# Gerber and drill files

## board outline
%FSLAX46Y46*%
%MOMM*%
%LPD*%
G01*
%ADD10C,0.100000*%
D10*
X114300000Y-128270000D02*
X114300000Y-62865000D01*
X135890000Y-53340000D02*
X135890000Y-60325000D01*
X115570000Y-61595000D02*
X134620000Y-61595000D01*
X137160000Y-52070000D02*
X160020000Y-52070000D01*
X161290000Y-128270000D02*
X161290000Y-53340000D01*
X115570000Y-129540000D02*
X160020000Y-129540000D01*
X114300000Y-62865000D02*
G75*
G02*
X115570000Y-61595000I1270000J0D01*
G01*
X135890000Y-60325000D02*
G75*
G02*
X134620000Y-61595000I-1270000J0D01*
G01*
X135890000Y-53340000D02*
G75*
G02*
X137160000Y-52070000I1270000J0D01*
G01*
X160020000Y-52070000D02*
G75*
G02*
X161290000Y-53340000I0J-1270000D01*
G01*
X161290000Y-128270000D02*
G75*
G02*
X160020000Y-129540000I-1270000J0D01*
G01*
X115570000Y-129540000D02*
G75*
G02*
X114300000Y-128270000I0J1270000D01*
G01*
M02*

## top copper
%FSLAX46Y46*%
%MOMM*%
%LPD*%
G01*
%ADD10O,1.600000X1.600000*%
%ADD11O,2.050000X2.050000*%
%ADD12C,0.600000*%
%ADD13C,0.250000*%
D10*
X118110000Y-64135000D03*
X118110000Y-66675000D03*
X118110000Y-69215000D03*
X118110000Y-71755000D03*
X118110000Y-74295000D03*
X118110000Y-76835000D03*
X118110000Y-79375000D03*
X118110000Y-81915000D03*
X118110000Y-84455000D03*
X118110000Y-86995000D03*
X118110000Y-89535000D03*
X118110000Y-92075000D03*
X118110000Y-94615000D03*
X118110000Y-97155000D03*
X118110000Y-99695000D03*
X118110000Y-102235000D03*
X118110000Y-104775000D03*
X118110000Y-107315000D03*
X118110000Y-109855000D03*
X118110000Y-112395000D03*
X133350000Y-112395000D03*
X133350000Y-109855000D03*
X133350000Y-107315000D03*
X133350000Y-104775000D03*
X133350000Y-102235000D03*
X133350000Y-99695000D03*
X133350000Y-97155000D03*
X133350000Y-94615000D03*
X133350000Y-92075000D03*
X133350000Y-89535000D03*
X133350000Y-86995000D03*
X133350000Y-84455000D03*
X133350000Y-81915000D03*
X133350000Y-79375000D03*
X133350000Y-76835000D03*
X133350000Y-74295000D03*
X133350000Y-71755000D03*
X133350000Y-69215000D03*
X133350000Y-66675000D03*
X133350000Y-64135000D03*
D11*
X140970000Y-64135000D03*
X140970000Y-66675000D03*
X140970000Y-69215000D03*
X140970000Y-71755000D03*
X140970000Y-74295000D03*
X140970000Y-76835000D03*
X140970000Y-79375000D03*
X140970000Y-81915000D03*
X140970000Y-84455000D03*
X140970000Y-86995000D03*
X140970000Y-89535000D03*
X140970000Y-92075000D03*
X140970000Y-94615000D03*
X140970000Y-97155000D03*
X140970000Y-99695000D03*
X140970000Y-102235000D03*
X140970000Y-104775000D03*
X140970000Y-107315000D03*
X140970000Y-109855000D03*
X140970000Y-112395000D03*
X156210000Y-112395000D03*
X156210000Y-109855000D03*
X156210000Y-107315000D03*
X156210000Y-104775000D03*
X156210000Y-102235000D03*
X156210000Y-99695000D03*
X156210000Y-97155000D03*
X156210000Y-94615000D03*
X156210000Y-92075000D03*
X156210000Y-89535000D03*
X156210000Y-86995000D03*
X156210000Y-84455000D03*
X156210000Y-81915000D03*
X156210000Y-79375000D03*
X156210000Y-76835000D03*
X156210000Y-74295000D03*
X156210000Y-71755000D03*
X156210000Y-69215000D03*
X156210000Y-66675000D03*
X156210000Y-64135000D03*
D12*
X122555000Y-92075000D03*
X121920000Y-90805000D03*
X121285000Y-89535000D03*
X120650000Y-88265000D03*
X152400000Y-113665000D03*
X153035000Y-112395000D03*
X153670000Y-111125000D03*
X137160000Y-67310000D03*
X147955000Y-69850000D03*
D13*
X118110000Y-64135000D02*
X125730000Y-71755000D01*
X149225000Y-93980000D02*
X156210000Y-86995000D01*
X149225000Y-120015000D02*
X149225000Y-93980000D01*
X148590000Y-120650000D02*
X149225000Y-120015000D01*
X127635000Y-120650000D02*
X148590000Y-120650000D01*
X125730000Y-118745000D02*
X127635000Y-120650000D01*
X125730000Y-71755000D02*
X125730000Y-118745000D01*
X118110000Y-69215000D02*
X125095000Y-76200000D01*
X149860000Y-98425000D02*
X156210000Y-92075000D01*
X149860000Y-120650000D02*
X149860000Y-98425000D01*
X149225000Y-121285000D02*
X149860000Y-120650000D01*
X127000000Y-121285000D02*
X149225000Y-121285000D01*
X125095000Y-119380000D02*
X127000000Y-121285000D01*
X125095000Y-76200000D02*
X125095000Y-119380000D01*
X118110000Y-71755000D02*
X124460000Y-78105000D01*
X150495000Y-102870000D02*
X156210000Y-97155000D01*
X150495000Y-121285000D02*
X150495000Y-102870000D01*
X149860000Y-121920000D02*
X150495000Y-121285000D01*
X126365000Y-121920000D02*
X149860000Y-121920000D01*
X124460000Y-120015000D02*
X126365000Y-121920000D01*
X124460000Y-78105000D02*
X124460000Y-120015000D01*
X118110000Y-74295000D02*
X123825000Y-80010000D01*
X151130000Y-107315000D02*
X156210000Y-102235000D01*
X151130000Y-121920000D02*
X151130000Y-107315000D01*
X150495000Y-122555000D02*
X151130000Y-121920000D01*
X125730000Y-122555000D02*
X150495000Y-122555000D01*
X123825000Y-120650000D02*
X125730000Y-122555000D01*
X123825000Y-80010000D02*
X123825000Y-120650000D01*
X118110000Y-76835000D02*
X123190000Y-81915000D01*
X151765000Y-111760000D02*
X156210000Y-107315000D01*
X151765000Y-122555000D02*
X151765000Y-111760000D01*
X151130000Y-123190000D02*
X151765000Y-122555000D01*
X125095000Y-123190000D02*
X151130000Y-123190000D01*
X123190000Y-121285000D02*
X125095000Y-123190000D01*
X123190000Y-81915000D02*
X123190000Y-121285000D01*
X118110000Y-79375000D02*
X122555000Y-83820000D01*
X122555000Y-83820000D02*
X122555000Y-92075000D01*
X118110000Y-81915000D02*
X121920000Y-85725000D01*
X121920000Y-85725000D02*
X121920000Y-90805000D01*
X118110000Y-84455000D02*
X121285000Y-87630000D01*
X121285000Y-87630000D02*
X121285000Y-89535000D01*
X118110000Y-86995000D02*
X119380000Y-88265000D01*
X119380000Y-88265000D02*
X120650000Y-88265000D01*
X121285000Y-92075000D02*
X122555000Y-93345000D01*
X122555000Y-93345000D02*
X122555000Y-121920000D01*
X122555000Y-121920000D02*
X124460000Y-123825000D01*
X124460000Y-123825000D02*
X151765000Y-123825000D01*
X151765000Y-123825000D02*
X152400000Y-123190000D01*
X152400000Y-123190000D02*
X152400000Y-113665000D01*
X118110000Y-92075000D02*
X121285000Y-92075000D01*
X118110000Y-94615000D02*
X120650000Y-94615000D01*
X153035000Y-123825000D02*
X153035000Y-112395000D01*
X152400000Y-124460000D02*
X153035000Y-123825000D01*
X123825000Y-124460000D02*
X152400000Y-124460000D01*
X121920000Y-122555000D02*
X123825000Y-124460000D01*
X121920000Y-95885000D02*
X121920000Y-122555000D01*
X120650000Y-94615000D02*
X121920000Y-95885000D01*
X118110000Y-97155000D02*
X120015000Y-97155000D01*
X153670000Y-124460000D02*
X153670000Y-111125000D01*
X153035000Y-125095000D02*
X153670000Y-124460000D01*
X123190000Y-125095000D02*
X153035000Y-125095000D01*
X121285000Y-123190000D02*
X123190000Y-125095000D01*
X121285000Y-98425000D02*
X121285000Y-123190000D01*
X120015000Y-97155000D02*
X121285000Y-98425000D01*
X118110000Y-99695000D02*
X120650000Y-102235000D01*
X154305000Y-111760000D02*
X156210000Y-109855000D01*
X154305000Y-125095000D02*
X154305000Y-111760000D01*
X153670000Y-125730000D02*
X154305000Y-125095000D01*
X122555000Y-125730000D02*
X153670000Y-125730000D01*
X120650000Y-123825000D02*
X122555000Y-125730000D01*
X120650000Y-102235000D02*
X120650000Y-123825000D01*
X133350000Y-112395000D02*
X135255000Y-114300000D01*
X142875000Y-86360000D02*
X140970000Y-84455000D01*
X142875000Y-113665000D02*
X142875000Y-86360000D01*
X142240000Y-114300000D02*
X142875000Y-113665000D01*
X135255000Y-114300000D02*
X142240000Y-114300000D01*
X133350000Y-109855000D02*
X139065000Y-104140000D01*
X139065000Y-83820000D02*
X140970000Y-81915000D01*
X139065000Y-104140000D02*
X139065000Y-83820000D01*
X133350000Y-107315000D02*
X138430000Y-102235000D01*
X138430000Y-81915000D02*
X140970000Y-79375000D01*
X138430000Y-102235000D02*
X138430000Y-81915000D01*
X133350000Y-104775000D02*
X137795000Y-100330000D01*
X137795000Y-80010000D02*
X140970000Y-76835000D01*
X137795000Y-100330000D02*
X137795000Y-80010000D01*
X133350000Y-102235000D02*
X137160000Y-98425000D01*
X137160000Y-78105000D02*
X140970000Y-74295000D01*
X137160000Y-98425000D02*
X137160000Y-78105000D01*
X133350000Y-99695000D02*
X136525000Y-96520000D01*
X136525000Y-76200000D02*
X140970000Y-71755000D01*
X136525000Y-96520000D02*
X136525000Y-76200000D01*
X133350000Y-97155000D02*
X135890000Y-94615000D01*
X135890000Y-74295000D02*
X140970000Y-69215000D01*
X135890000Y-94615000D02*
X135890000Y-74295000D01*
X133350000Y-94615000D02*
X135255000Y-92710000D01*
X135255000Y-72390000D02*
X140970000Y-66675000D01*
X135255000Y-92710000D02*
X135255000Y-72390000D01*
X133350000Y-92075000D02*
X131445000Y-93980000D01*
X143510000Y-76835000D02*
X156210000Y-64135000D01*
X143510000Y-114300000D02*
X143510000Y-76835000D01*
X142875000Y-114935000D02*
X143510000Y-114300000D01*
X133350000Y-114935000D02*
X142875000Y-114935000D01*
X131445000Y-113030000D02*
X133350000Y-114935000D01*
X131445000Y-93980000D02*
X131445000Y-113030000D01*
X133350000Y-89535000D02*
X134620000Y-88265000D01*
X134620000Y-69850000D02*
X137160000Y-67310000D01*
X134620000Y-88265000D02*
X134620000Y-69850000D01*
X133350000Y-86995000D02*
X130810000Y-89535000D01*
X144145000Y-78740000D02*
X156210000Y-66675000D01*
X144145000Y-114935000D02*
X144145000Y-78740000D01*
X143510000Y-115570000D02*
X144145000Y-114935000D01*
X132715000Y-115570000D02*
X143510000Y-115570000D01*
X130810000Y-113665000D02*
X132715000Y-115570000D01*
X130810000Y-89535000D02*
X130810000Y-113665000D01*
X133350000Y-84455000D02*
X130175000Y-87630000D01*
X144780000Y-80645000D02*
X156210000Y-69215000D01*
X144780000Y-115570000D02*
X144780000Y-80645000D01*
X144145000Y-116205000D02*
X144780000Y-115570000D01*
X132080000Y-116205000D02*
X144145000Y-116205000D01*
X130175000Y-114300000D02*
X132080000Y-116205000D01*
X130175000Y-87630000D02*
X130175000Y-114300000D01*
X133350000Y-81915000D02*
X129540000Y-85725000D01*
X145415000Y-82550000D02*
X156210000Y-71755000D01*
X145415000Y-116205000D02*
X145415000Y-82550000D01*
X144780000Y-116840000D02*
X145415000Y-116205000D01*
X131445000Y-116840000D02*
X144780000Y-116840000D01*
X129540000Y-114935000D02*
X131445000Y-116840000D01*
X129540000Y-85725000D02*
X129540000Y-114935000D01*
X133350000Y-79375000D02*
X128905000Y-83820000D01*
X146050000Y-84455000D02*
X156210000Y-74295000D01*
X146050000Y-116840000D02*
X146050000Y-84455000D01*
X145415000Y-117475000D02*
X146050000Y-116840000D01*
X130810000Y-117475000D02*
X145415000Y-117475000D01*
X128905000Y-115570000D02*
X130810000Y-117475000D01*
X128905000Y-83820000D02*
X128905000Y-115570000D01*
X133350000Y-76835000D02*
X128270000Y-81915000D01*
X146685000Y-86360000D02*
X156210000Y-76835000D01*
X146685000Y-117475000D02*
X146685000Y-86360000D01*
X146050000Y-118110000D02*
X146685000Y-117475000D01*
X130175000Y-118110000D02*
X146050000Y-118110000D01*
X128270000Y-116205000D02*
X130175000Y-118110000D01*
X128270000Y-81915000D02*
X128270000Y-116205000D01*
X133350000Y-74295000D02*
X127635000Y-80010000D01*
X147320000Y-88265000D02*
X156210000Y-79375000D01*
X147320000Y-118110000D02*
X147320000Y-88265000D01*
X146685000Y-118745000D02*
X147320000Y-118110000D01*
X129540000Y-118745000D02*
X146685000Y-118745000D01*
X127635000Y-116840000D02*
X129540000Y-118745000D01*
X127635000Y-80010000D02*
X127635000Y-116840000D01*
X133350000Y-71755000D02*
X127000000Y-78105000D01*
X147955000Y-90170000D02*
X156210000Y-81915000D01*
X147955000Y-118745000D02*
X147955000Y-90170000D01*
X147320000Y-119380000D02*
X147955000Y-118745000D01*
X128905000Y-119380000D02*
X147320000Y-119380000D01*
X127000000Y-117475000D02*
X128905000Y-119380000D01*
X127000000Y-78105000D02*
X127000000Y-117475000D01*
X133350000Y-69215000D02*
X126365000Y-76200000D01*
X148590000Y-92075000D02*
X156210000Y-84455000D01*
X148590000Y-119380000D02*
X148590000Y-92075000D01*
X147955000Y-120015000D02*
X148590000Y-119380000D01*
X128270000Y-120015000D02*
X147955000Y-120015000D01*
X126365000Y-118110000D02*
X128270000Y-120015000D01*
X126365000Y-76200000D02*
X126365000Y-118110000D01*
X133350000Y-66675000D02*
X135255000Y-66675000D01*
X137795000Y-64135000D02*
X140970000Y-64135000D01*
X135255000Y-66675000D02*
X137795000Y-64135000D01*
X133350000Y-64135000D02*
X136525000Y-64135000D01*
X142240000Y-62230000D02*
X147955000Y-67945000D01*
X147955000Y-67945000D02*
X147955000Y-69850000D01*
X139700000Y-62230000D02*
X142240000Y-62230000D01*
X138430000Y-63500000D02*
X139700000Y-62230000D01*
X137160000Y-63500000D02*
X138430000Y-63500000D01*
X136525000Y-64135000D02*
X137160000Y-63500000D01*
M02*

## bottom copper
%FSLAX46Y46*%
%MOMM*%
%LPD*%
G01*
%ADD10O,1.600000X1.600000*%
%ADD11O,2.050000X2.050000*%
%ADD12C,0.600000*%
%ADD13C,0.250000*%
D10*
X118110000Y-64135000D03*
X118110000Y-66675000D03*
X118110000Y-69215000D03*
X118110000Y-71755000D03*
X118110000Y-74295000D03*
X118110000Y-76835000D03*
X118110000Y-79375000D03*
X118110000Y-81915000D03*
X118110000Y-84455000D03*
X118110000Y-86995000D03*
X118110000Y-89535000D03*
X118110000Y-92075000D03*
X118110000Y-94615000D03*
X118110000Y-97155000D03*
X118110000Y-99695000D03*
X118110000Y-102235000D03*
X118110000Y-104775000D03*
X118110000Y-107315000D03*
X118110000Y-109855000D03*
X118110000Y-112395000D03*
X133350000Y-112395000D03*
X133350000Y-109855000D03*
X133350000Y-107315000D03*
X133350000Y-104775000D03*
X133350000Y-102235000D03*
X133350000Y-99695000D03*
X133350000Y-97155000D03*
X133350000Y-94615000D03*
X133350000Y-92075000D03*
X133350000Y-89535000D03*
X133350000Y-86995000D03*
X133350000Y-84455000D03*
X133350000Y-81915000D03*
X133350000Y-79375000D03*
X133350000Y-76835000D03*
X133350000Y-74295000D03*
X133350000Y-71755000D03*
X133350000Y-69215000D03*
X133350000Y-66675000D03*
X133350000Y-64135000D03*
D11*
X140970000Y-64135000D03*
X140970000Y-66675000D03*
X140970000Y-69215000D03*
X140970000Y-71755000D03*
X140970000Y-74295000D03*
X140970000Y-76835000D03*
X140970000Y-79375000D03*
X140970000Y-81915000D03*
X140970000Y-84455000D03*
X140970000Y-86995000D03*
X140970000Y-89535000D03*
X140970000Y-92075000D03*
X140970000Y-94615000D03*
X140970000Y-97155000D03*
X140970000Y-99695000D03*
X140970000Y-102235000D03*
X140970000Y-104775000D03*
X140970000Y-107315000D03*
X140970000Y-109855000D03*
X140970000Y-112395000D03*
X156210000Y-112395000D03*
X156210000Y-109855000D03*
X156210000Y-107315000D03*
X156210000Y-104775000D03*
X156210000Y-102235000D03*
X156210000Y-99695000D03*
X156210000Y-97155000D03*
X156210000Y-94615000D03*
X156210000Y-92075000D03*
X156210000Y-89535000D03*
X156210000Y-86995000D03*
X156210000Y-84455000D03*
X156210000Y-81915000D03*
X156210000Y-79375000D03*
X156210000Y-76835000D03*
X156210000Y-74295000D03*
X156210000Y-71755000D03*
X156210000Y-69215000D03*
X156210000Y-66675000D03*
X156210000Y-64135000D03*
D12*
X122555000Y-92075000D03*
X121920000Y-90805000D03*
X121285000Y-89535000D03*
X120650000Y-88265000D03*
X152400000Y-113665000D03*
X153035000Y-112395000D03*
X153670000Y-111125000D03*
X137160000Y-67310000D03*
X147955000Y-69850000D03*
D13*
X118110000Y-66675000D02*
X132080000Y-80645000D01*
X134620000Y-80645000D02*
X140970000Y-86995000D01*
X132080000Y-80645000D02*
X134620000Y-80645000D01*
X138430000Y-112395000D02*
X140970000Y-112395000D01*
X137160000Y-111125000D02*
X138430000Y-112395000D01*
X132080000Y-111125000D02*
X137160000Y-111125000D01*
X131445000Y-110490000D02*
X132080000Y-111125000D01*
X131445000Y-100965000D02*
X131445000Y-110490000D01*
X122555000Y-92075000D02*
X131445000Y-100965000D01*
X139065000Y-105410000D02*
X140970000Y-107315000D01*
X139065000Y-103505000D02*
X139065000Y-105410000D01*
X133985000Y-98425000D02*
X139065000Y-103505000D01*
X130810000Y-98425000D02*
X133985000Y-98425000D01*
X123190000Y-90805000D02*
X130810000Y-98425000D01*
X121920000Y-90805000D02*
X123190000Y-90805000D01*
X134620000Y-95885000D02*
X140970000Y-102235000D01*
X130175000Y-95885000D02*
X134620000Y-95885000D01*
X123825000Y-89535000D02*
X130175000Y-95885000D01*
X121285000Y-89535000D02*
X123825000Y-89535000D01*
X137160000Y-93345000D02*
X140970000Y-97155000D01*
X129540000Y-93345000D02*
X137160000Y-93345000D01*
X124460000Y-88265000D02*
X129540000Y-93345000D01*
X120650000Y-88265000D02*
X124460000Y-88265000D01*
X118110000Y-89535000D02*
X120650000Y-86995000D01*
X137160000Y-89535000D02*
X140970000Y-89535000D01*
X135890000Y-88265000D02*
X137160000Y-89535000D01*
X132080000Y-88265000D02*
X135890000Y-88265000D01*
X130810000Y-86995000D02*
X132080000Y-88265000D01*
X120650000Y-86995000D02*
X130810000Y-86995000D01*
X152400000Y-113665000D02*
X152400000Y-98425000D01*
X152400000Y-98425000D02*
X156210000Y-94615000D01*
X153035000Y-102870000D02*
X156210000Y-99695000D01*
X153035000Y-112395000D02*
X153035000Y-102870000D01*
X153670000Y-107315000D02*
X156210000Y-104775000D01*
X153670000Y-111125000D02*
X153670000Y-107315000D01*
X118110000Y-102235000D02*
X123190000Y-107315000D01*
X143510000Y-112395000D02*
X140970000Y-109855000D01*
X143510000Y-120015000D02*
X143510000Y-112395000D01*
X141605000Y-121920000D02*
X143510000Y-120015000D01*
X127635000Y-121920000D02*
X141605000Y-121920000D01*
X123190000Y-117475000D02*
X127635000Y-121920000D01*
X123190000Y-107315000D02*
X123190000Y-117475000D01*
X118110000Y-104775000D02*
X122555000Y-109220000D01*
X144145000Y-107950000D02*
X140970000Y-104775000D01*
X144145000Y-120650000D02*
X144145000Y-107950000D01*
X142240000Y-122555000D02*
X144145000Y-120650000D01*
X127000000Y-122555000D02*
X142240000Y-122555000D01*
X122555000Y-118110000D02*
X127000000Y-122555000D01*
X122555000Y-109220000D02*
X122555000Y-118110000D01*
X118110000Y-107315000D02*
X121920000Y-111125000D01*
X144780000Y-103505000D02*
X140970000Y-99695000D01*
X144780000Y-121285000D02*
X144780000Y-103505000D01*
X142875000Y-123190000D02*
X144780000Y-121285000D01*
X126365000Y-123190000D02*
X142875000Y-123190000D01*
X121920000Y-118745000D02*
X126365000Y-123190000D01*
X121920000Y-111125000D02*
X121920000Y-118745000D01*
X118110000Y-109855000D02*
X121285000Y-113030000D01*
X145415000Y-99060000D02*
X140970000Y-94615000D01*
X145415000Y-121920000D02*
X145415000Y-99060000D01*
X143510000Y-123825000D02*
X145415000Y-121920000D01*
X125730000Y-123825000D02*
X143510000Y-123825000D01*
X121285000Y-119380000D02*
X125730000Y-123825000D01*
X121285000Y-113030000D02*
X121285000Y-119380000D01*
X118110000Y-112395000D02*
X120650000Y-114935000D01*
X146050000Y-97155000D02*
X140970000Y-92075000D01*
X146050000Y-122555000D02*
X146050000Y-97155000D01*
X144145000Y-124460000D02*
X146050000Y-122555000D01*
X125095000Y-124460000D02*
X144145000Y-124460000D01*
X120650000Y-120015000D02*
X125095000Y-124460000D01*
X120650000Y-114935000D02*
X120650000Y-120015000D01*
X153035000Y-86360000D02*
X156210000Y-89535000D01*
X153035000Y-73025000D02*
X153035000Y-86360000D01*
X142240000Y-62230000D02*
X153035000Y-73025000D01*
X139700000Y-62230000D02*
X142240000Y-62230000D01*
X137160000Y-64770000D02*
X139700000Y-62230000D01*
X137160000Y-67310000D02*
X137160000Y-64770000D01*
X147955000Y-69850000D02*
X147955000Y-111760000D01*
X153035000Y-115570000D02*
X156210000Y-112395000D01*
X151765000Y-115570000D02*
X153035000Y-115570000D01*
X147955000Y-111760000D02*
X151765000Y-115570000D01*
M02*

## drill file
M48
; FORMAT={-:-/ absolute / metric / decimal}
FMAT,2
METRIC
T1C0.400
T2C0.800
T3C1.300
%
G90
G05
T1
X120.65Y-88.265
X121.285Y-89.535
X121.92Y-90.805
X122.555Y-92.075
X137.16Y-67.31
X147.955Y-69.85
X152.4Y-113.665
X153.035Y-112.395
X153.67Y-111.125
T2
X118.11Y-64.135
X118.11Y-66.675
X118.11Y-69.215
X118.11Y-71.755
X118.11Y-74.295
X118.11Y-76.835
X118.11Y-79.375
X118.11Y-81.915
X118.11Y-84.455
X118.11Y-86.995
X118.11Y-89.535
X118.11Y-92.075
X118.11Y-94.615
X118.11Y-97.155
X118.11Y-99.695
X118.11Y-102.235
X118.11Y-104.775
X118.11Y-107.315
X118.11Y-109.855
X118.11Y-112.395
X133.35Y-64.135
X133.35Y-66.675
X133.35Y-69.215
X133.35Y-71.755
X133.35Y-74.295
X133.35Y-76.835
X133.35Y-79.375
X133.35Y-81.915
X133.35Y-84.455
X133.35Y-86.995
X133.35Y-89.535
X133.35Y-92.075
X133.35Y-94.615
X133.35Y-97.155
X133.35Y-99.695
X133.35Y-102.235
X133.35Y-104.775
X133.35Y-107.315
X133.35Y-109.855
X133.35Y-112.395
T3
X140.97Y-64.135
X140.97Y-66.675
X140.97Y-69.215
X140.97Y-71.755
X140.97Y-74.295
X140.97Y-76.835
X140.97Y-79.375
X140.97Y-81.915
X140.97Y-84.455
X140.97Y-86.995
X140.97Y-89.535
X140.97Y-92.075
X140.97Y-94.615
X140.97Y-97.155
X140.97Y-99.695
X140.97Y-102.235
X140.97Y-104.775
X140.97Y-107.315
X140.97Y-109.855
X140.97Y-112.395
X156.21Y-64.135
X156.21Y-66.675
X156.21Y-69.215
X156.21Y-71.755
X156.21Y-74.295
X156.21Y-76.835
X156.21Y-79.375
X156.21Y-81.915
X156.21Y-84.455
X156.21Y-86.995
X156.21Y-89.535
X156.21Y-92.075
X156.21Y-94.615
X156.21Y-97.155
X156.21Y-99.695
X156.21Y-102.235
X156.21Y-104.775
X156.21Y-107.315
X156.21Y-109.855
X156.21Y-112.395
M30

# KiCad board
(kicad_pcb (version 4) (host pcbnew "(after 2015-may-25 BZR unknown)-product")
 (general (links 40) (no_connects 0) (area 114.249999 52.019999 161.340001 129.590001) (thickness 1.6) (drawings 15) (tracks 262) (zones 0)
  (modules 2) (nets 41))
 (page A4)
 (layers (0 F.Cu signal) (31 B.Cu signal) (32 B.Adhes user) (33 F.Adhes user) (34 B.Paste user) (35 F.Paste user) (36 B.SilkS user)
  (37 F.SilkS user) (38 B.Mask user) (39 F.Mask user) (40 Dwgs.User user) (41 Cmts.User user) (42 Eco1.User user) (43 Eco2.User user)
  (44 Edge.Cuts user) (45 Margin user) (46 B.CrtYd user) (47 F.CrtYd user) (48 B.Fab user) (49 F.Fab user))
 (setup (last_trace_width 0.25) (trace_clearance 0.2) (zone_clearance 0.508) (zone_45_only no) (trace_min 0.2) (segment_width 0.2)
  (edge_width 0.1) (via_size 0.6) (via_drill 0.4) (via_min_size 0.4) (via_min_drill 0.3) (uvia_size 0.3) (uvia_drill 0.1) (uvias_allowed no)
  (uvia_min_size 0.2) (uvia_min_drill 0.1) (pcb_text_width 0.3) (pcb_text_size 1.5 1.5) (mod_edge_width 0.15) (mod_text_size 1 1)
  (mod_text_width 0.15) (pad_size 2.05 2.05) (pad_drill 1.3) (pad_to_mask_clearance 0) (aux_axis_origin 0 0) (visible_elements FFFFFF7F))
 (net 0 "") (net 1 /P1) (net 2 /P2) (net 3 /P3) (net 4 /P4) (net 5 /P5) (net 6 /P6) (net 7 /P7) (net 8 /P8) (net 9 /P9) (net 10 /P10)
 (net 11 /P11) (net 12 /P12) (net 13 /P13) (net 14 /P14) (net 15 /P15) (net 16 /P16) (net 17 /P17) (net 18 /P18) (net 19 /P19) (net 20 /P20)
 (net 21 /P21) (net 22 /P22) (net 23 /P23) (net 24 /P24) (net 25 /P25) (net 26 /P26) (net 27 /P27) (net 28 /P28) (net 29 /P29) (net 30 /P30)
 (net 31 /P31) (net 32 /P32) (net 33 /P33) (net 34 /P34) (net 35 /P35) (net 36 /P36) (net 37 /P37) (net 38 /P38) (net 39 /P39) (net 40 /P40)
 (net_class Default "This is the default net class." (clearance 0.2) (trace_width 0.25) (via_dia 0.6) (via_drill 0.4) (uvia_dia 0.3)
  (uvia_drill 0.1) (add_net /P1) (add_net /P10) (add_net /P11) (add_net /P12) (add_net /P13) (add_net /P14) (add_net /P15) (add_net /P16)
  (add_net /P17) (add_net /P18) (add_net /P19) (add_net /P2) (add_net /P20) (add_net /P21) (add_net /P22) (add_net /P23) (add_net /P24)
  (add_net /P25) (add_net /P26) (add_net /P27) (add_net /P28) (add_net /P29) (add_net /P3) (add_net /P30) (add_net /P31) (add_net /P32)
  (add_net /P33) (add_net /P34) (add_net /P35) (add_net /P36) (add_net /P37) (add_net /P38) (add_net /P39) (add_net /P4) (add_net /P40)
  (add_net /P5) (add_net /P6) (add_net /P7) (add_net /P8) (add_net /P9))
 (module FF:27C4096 (layer F.Cu) (at 118.11 64.135)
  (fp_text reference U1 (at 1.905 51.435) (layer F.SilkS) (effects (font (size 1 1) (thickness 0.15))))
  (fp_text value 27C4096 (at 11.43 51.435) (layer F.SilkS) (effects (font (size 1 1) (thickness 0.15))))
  (pad 1 thru_hole oval (at 0 0) (size 1.6 1.6) (drill 0.8) (layers *.Cu *.Mask F.SilkS) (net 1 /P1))
  (pad 2 thru_hole oval (at 0 2.54) (size 1.6 1.6) (drill 0.8) (layers *.Cu *.Mask F.SilkS) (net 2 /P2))
  (pad 3 thru_hole oval (at 0 5.08) (size 1.6 1.6) (drill 0.8) (layers *.Cu *.Mask F.SilkS) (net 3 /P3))
  (pad 4 thru_hole oval (at 0 7.62) (size 1.6 1.6) (drill 0.8) (layers *.Cu *.Mask F.SilkS) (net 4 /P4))
  (pad 5 thru_hole oval (at 0 10.16) (size 1.6 1.6) (drill 0.8) (layers *.Cu *.Mask F.SilkS) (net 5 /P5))
  (pad 6 thru_hole oval (at 0 12.7) (size 1.6 1.6) (drill 0.8) (layers *.Cu *.Mask F.SilkS) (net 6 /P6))
  (pad 7 thru_hole oval (at 0 15.24) (size 1.6 1.6) (drill 0.8) (layers *.Cu *.Mask F.SilkS) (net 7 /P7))
  (pad 8 thru_hole oval (at 0 17.78) (size 1.6 1.6) (drill 0.8) (layers *.Cu *.Mask F.SilkS) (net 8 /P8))
  (pad 9 thru_hole oval (at 0 20.32) (size 1.6 1.6) (drill 0.8) (layers *.Cu *.Mask F.SilkS) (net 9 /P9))
  (pad 10 thru_hole oval (at 0 22.86) (size 1.6 1.6) (drill 0.8) (layers *.Cu *.Mask F.SilkS) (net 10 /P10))
  (pad 11 thru_hole oval (at 0 25.4) (size 1.6 1.6) (drill 0.8) (layers *.Cu *.Mask F.SilkS) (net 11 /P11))
  (pad 12 thru_hole oval (at 0 27.94) (size 1.6 1.6) (drill 0.8) (layers *.Cu *.Mask F.SilkS) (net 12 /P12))
  (pad 13 thru_hole oval (at 0 30.48) (size 1.6 1.6) (drill 0.8) (layers *.Cu *.Mask F.SilkS) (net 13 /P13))
  (pad 14 thru_hole oval (at 0 33.02) (size 1.6 1.6) (drill 0.8) (layers *.Cu *.Mask F.SilkS) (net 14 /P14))
  (pad 15 thru_hole oval (at 0 35.56) (size 1.6 1.6) (drill 0.8) (layers *.Cu *.Mask F.SilkS) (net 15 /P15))
  (pad 16 thru_hole oval (at 0 38.1) (size 1.6 1.6) (drill 0.8) (layers *.Cu *.Mask F.SilkS) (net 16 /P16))
  (pad 17 thru_hole oval (at 0 40.64) (size 1.6 1.6) (drill 0.8) (layers *.Cu *.Mask F.SilkS) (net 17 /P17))
  (pad 18 thru_hole oval (at 0 43.18) (size 1.6 1.6) (drill 0.8) (layers *.Cu *.Mask F.SilkS) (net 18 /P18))
  (pad 19 thru_hole oval (at 0 45.72) (size 1.6 1.6) (drill 0.8) (layers *.Cu *.Mask F.SilkS) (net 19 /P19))
  (pad 20 thru_hole oval (at 0 48.26) (size 1.6 1.6) (drill 0.8) (layers *.Cu *.Mask F.SilkS) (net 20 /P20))
  (pad 21 thru_hole oval (at 15.24 48.26) (size 1.6 1.6) (drill 0.8) (layers *.Cu *.Mask F.SilkS) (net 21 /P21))
  (pad 22 thru_hole oval (at 15.24 45.72) (size 1.6 1.6) (drill 0.8) (layers *.Cu *.Mask F.SilkS) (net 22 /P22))
  (pad 23 thru_hole oval (at 15.24 43.18) (size 1.6 1.6) (drill 0.8) (layers *.Cu *.Mask F.SilkS) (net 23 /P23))
  (pad 24 thru_hole oval (at 15.24 40.64) (size 1.6 1.6) (drill 0.8) (layers *.Cu *.Mask F.SilkS) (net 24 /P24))
  (pad 25 thru_hole oval (at 15.24 38.1) (size 1.6 1.6) (drill 0.8) (layers *.Cu *.Mask F.SilkS) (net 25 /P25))
  (pad 26 thru_hole oval (at 15.24 35.56) (size 1.6 1.6) (drill 0.8) (layers *.Cu *.Mask F.SilkS) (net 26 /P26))
  (pad 27 thru_hole oval (at 15.24 33.02) (size 1.6 1.6) (drill 0.8) (layers *.Cu *.Mask F.SilkS) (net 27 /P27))
  (pad 28 thru_hole oval (at 15.24 30.48) (size 1.6 1.6) (drill 0.8) (layers *.Cu *.Mask F.SilkS) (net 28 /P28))
  (pad 29 thru_hole oval (at 15.24 27.94) (size 1.6 1.6) (drill 0.8) (layers *.Cu *.Mask F.SilkS) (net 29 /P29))
  (pad 30 thru_hole oval (at 15.24 25.4) (size 1.6 1.6) (drill 0.8) (layers *.Cu *.Mask F.SilkS) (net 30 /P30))
  (pad 31 thru_hole oval (at 15.24 22.86) (size 1.6 1.6) (drill 0.8) (layers *.Cu *.Mask F.SilkS) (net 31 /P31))
  (pad 32 thru_hole oval (at 15.24 20.32) (size 1.6 1.6) (drill 0.8) (layers *.Cu *.Mask F.SilkS) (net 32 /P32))
  (pad 33 thru_hole oval (at 15.24 17.78) (size 1.6 1.6) (drill 0.8) (layers *.Cu *.Mask F.SilkS) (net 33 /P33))
  (pad 34 thru_hole oval (at 15.24 15.24) (size 1.6 1.6) (drill 0.8) (layers *.Cu *.Mask F.SilkS) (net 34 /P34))
  (pad 35 thru_hole oval (at 15.24 12.7) (size 1.6 1.6) (drill 0.8) (layers *.Cu *.Mask F.SilkS) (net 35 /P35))
  (pad 36 thru_hole oval (at 15.24 10.16) (size 1.6 1.6) (drill 0.8) (layers *.Cu *.Mask F.SilkS) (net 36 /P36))
  (pad 37 thru_hole oval (at 15.24 7.62) (size 1.6 1.6) (drill 0.8) (layers *.Cu *.Mask F.SilkS) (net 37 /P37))
  (pad 38 thru_hole oval (at 15.24 5.08) (size 1.6 1.6) (drill 0.8) (layers *.Cu *.Mask F.SilkS) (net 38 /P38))
  (pad 39 thru_hole oval (at 15.24 2.54) (size 1.6 1.6) (drill 0.8) (layers *.Cu *.Mask F.SilkS) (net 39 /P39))
  (pad 40 thru_hole oval (at 15.24 0) (size 1.6 1.6) (drill 0.8) (layers *.Cu *.Mask F.SilkS) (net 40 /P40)))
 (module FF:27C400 (layer F.Cu) (at 140.97 64.135)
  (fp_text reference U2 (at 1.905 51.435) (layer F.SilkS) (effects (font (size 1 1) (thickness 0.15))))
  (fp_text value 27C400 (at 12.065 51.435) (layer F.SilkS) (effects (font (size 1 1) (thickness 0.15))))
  (pad 1 thru_hole oval (at 0 0) (size 2.05 2.05) (drill 1.3) (layers *.Cu *.Mask F.SilkS) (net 39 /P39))
  (pad 2 thru_hole oval (at 0 2.54) (size 2.05 2.05) (drill 1.3) (layers *.Cu *.Mask F.SilkS) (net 28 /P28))
  (pad 3 thru_hole oval (at 0 5.08) (size 2.05 2.05) (drill 1.3) (layers *.Cu *.Mask F.SilkS) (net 27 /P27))
  (pad 4 thru_hole oval (at 0 7.62) (size 2.05 2.05) (drill 1.3) (layers *.Cu *.Mask F.SilkS) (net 26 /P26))
  (pad 5 thru_hole oval (at 0 10.16) (size 2.05 2.05) (drill 1.3) (layers *.Cu *.Mask F.SilkS) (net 25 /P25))
  (pad 6 thru_hole oval (at 0 12.7) (size 2.05 2.05) (drill 1.3) (layers *.Cu *.Mask F.SilkS) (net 24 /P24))
  (pad 7 thru_hole oval (at 0 15.24) (size 2.05 2.05) (drill 1.3) (layers *.Cu *.Mask F.SilkS) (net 23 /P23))
  (pad 8 thru_hole oval (at 0 17.78) (size 2.05 2.05) (drill 1.3) (layers *.Cu *.Mask F.SilkS) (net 22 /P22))
  (pad 9 thru_hole oval (at 0 20.32) (size 2.05 2.05) (drill 1.3) (layers *.Cu *.Mask F.SilkS) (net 21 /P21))
  (pad 10 thru_hole oval (at 0 22.86) (size 2.05 2.05) (drill 1.3) (layers *.Cu *.Mask F.SilkS) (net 2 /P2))
  (pad 11 thru_hole oval (at 0 25.4) (size 2.05 2.05) (drill 1.3) (layers *.Cu *.Mask F.SilkS) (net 11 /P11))
  (pad 12 thru_hole oval (at 0 27.94) (size 2.05 2.05) (drill 1.3) (layers *.Cu *.Mask F.SilkS) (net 20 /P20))
  (pad 13 thru_hole oval (at 0 30.48) (size 2.05 2.05) (drill 1.3) (layers *.Cu *.Mask F.SilkS) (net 19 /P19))
  (pad 14 thru_hole oval (at 0 33.02) (size 2.05 2.05) (drill 1.3) (layers *.Cu *.Mask F.SilkS) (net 10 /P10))
  (pad 15 thru_hole oval (at 0 35.56) (size 2.05 2.05) (drill 1.3) (layers *.Cu *.Mask F.SilkS) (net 18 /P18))
  (pad 16 thru_hole oval (at 0 38.1) (size 2.05 2.05) (drill 1.3) (layers *.Cu *.Mask F.SilkS) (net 9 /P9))
  (pad 17 thru_hole oval (at 0 40.64) (size 2.05 2.05) (drill 1.3) (layers *.Cu *.Mask F.SilkS) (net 17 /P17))
  (pad 18 thru_hole oval (at 0 43.18) (size 2.05 2.05) (drill 1.3) (layers *.Cu *.Mask F.SilkS) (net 8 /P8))
  (pad 19 thru_hole oval (at 0 45.72) (size 2.05 2.05) (drill 1.3) (layers *.Cu *.Mask F.SilkS) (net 16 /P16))
  (pad 20 thru_hole oval (at 0 48.26) (size 2.05 2.05) (drill 1.3) (layers *.Cu *.Mask F.SilkS) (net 7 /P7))
  (pad 21 thru_hole oval (at 15.24 48.26) (size 2.05 2.05) (drill 1.3) (layers *.Cu *.Mask F.SilkS) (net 40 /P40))
  (pad 22 thru_hole oval (at 15.24 45.72) (size 2.05 2.05) (drill 1.3) (layers *.Cu *.Mask F.SilkS) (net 15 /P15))
  (pad 23 thru_hole oval (at 15.24 43.18) (size 2.05 2.05) (drill 1.3) (layers *.Cu *.Mask F.SilkS) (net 6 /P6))
  (pad 24 thru_hole oval (at 15.24 40.64) (size 2.05 2.05) (drill 1.3) (layers *.Cu *.Mask F.SilkS) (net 14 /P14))
  (pad 25 thru_hole oval (at 15.24 38.1) (size 2.05 2.05) (drill 1.3) (layers *.Cu *.Mask F.SilkS) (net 5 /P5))
  (pad 26 thru_hole oval (at 15.24 35.56) (size 2.05 2.05) (drill 1.3) (layers *.Cu *.Mask F.SilkS) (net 13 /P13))
  (pad 27 thru_hole oval (at 15.24 33.02) (size 2.05 2.05) (drill 1.3) (layers *.Cu *.Mask F.SilkS) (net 4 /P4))
  (pad 28 thru_hole oval (at 15.24 30.48) (size 2.05 2.05) (drill 1.3) (layers *.Cu *.Mask F.SilkS) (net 12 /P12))
  (pad 29 thru_hole oval (at 15.24 27.94) (size 2.05 2.05) (drill 1.3) (layers *.Cu *.Mask F.SilkS) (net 3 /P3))
  (pad 30 thru_hole oval (at 15.24 25.4) (size 2.05 2.05) (drill 1.3) (layers *.Cu *.Mask F.SilkS) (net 30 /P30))
  (pad 31 thru_hole oval (at 15.24 22.86) (size 2.05 2.05) (drill 1.3) (layers *.Cu *.Mask F.SilkS) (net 1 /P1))
  (pad 32 thru_hole oval (at 15.24 20.32) (size 2.05 2.05) (drill 1.3) (layers *.Cu *.Mask F.SilkS) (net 38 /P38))
  (pad 33 thru_hole oval (at 15.24 17.78) (size 2.05 2.05) (drill 1.3) (layers *.Cu *.Mask F.SilkS) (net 37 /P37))
  (pad 34 thru_hole oval (at 15.24 15.24) (size 2.05 2.05) (drill 1.3) (layers *.Cu *.Mask F.SilkS) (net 36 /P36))
  (pad 35 thru_hole oval (at 15.24 12.7) (size 2.05 2.05) (drill 1.3) (layers *.Cu *.Mask F.SilkS) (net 35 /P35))
  (pad 36 thru_hole oval (at 15.24 10.16) (size 2.05 2.05) (drill 1.3) (layers *.Cu *.Mask F.SilkS) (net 34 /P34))
  (pad 37 thru_hole oval (at 15.24 7.62) (size 2.05 2.05) (drill 1.3) (layers *.Cu *.Mask F.SilkS) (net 33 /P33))
  (pad 38 thru_hole oval (at 15.24 5.08) (size 2.05 2.05) (drill 1.3) (layers *.Cu *.Mask F.SilkS) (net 32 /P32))
  (pad 39 thru_hole oval (at 15.24 2.54) (size 2.05 2.05) (drill 1.3) (layers *.Cu *.Mask F.SilkS) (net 31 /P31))
  (pad 40 thru_hole oval (at 15.24 0) (size 2.05 2.05) (drill 1.3) (layers *.Cu *.Mask F.SilkS) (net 29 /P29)))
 (gr_line (start 114.3 128.27) (end 114.3 62.865) (angle 90) (layer Edge.Cuts) (width 0.1))
 (gr_line (start 135.89 53.34) (end 135.89 60.325) (angle 90) (layer Edge.Cuts) (width 0.1))
 (gr_line (start 115.57 61.595) (end 134.62 61.595) (angle 90) (layer Edge.Cuts) (width 0.1))
 (gr_line (start 137.16 52.07) (end 160.02 52.07) (angle 90) (layer Edge.Cuts) (width 0.1))
 (gr_line (start 161.29 128.27) (end 161.29 53.34) (angle 90) (layer Edge.Cuts) (width 0.1))
 (gr_line (start 115.57 129.54) (end 160.02 129.54) (angle 90) (layer Edge.Cuts) (width 0.1))
 (gr_arc (start 115.57 62.865) (end 114.3 62.865) (angle 90) (layer Edge.Cuts) (width 0.1))
 (gr_arc (start 134.62 60.325) (end 135.89 60.325) (angle 90) (layer Edge.Cuts) (width 0.1))
 (gr_arc (start 137.16 53.34) (end 135.89 53.34) (angle 90) (layer Edge.Cuts) (width 0.1))
 (gr_arc (start 160.02 53.34) (end 160.02 52.07) (angle 90) (layer Edge.Cuts) (width 0.1))
 (gr_arc (start 160.02 128.27) (end 161.29 128.27) (angle 90) (layer Edge.Cuts) (width 0.1))
 (gr_arc (start 115.57 128.27) (end 115.57 129.54) (angle 90) (layer Edge.Cuts) (width 0.1))
 (segment (start 118.11 64.135) (end 125.73 71.755) (width 0.25) (layer F.Cu) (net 1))
 (segment (start 149.225 93.98) (end 156.21 86.995) (width 0.25) (layer F.Cu) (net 1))
 (segment (start 149.225 120.015) (end 149.225 93.98) (width 0.25) (layer F.Cu) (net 1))
 (segment (start 148.59 120.65) (end 149.225 120.015) (width 0.25) (layer F.Cu) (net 1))
 (segment (start 127.635 120.65) (end 148.59 120.65) (width 0.25) (layer F.Cu) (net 1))
 (segment (start 125.73 118.745) (end 127.635 120.65) (width 0.25) (layer F.Cu) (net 1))
 (segment (start 125.73 71.755) (end 125.73 118.745) (width 0.25) (layer F.Cu) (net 1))
 (segment (start 118.11 66.675) (end 132.08 80.645) (width 0.25) (layer B.Cu) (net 2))
 (segment (start 134.62 80.645) (end 140.97 86.995) (width 0.25) (layer B.Cu) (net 2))
 (segment (start 132.08 80.645) (end 134.62 80.645) (width 0.25) (layer B.Cu) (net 2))
 (segment (start 118.11 69.215) (end 125.095 76.2) (width 0.25) (layer F.Cu) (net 3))
 (segment (start 149.86 98.425) (end 156.21 92.075) (width 0.25) (layer F.Cu) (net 3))
 (segment (start 149.86 120.65) (end 149.86 98.425) (width 0.25) (layer F.Cu) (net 3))
 (segment (start 149.225 121.285) (end 149.86 120.65) (width 0.25) (layer F.Cu) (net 3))
 (segment (start 127 121.285) (end 149.225 121.285) (width 0.25) (layer F.Cu) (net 3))
 (segment (start 125.095 119.38) (end 127 121.285) (width 0.25) (layer F.Cu) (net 3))
 (segment (start 125.095 76.2) (end 125.095 119.38) (width 0.25) (layer F.Cu) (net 3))
 (segment (start 118.11 71.755) (end 124.46 78.105) (width 0.25) (layer F.Cu) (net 4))
 (segment (start 150.495 102.87) (end 156.21 97.155) (width 0.25) (layer F.Cu) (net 4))
 (segment (start 150.495 121.285) (end 150.495 102.87) (width 0.25) (layer F.Cu) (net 4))
 (segment (start 149.86 121.92) (end 150.495 121.285) (width 0.25) (layer F.Cu) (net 4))
 (segment (start 126.365 121.92) (end 149.86 121.92) (width 0.25) (layer F.Cu) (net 4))
 (segment (start 124.46 120.015) (end 126.365 121.92) (width 0.25) (layer F.Cu) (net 4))
 (segment (start 124.46 78.105) (end 124.46 120.015) (width 0.25) (layer F.Cu) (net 4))
 (segment (start 118.11 74.295) (end 123.825 80.01) (width 0.25) (layer F.Cu) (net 5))
 (segment (start 151.13 107.315) (end 156.21 102.235) (width 0.25) (layer F.Cu) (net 5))
 (segment (start 151.13 121.92) (end 151.13 107.315) (width 0.25) (layer F.Cu) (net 5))
 (segment (start 150.495 122.555) (end 151.13 121.92) (width 0.25) (layer F.Cu) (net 5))
 (segment (start 125.73 122.555) (end 150.495 122.555) (width 0.25) (layer F.Cu) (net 5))
 (segment (start 123.825 120.65) (end 125.73 122.555) (width 0.25) (layer F.Cu) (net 5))
 (segment (start 123.825 80.01) (end 123.825 120.65) (width 0.25) (layer F.Cu) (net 5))
 (segment (start 118.11 76.835) (end 123.19 81.915) (width 0.25) (layer F.Cu) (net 6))
 (segment (start 151.765 111.76) (end 156.21 107.315) (width 0.25) (layer F.Cu) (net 6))
 (segment (start 151.765 122.555) (end 151.765 111.76) (width 0.25) (layer F.Cu) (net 6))
 (segment (start 151.13 123.19) (end 151.765 122.555) (width 0.25) (layer F.Cu) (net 6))
 (segment (start 125.095 123.19) (end 151.13 123.19) (width 0.25) (layer F.Cu) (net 6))
 (segment (start 123.19 121.285) (end 125.095 123.19) (width 0.25) (layer F.Cu) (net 6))
 (segment (start 123.19 81.915) (end 123.19 121.285) (width 0.25) (layer F.Cu) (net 6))
 (segment (start 118.11 79.375) (end 122.555 83.82) (width 0.25) (layer F.Cu) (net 7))
 (segment (start 138.43 112.395) (end 140.97 112.395) (width 0.25) (layer B.Cu) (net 7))
 (segment (start 137.16 111.125) (end 138.43 112.395) (width 0.25) (layer B.Cu) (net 7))
 (segment (start 132.08 111.125) (end 137.16 111.125) (width 0.25) (layer B.Cu) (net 7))
 (segment (start 131.445 110.49) (end 132.08 111.125) (width 0.25) (layer B.Cu) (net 7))
 (segment (start 131.445 100.965) (end 131.445 110.49) (width 0.25) (layer B.Cu) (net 7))
 (segment (start 122.555 92.075) (end 131.445 100.965) (width 0.25) (layer B.Cu) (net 7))
 (via (at 122.555 92.075) (size 0.6) (drill 0.4) (layers F.Cu B.Cu) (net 7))
 (segment (start 122.555 83.82) (end 122.555 92.075) (width 0.25) (layer F.Cu) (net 7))
 (segment (start 118.11 81.915) (end 121.92 85.725) (width 0.25) (layer F.Cu) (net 8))
 (segment (start 139.065 105.41) (end 140.97 107.315) (width 0.25) (layer B.Cu) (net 8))
 (segment (start 139.065 103.505) (end 139.065 105.41) (width 0.25) (layer B.Cu) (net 8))
 (segment (start 133.985 98.425) (end 139.065 103.505) (width 0.25) (layer B.Cu) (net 8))
 (segment (start 130.81 98.425) (end 133.985 98.425) (width 0.25) (layer B.Cu) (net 8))
 (segment (start 123.19 90.805) (end 130.81 98.425) (width 0.25) (layer B.Cu) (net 8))
 (segment (start 121.92 90.805) (end 123.19 90.805) (width 0.25) (layer B.Cu) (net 8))
 (via (at 121.92 90.805) (size 0.6) (drill 0.4) (layers F.Cu B.Cu) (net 8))
 (segment (start 121.92 85.725) (end 121.92 90.805) (width 0.25) (layer F.Cu) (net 8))
 (segment (start 118.11 84.455) (end 121.285 87.63) (width 0.25) (layer F.Cu) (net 9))
 (segment (start 134.62 95.885) (end 140.97 102.235) (width 0.25) (layer B.Cu) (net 9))
 (segment (start 130.175 95.885) (end 134.62 95.885) (width 0.25) (layer B.Cu) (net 9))
 (segment (start 123.825 89.535) (end 130.175 95.885) (width 0.25) (layer B.Cu) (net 9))
 (segment (start 121.285 89.535) (end 123.825 89.535) (width 0.25) (layer B.Cu) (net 9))
 (via (at 121.285 89.535) (size 0.6) (drill 0.4) (layers F.Cu B.Cu) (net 9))
 (segment (start 121.285 87.63) (end 121.285 89.535) (width 0.25) (layer F.Cu) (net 9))
 (segment (start 118.11 86.995) (end 119.38 88.265) (width 0.25) (layer F.Cu) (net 10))
 (segment (start 137.16 93.345) (end 140.97 97.155) (width 0.25) (layer B.Cu) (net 10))
 (segment (start 129.54 93.345) (end 137.16 93.345) (width 0.25) (layer B.Cu) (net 10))
 (segment (start 124.46 88.265) (end 129.54 93.345) (width 0.25) (layer B.Cu) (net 10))
 (segment (start 120.65 88.265) (end 124.46 88.265) (width 0.25) (layer B.Cu) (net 10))
 (via (at 120.65 88.265) (size 0.6) (drill 0.4) (layers F.Cu B.Cu) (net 10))
 (segment (start 119.38 88.265) (end 120.65 88.265) (width 0.25) (layer F.Cu) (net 10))
 (segment (start 118.11 89.535) (end 120.65 86.995) (width 0.25) (layer B.Cu) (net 11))
 (segment (start 137.16 89.535) (end 140.97 89.535) (width 0.25) (layer B.Cu) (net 11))
 (segment (start 135.89 88.265) (end 137.16 89.535) (width 0.25) (layer B.Cu) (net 11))
 (segment (start 132.08 88.265) (end 135.89 88.265) (width 0.25) (layer B.Cu) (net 11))
 (segment (start 130.81 86.995) (end 132.08 88.265) (width 0.25) (layer B.Cu) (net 11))
 (segment (start 120.65 86.995) (end 130.81 86.995) (width 0.25) (layer B.Cu) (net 11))
 (segment (start 152.4 113.665) (end 152.4 98.425) (width 0.25) (layer B.Cu) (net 12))
 (segment (start 121.285 92.075) (end 122.555 93.345) (width 0.25) (layer F.Cu) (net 12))
 (segment (start 122.555 93.345) (end 122.555 121.92) (width 0.25) (layer F.Cu) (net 12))
 (segment (start 122.555 121.92) (end 124.46 123.825) (width 0.25) (layer F.Cu) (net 12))
 (segment (start 124.46 123.825) (end 151.765 123.825) (width 0.25) (layer F.Cu) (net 12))
 (segment (start 151.765 123.825) (end 152.4 123.19) (width 0.25) (layer F.Cu) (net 12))
 (segment (start 152.4 123.19) (end 152.4 113.665) (width 0.25) (layer F.Cu) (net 12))
 (via (at 152.4 113.665) (size 0.6) (drill 0.4) (layers F.Cu B.Cu) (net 12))
 (segment (start 118.11 92.075) (end 121.285 92.075) (width 0.25) (layer F.Cu) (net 12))
 (segment (start 152.4 98.425) (end 156.21 94.615) (width 0.25) (layer B.Cu) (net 12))
 (segment (start 118.11 94.615) (end 120.65 94.615) (width 0.25) (layer F.Cu) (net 13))
 (segment (start 153.035 102.87) (end 156.21 99.695) (width 0.25) (layer B.Cu) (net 13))
 (segment (start 153.035 112.395) (end 153.035 102.87) (width 0.25) (layer B.Cu) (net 13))
 (via (at 153.035 112.395) (size 0.6) (drill 0.4) (layers F.Cu B.Cu) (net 13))
 (segment (start 153.035 123.825) (end 153.035 112.395) (width 0.25) (layer F.Cu) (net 13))
 (segment (start 152.4 124.46) (end 153.035 123.825) (width 0.25) (layer F.Cu) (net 13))
 (segment (start 123.825 124.46) (end 152.4 124.46) (width 0.25) (layer F.Cu) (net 13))
 (segment (start 121.92 122.555) (end 123.825 124.46) (width 0.25) (layer F.Cu) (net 13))
 (segment (start 121.92 95.885) (end 121.92 122.555) (width 0.25) (layer F.Cu) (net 13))
 (segment (start 120.65 94.615) (end 121.92 95.885) (width 0.25) (layer F.Cu) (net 13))
 (segment (start 118.11 97.155) (end 120.015 97.155) (width 0.25) (layer F.Cu) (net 14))
 (segment (start 153.67 107.315) (end 156.21 104.775) (width 0.25) (layer B.Cu) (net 14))
 (segment (start 153.67 111.125) (end 153.67 107.315) (width 0.25) (layer B.Cu) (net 14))
 (via (at 153.67 111.125) (size 0.6) (drill 0.4) (layers F.Cu B.Cu) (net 14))
 (segment (start 153.67 124.46) (end 153.67 111.125) (width 0.25) (layer F.Cu) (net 14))
 (segment (start 153.035 125.095) (end 153.67 124.46) (width 0.25) (layer F.Cu) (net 14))
 (segment (start 123.19 125.095) (end 153.035 125.095) (width 0.25) (layer F.Cu) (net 14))
 (segment (start 121.285 123.19) (end 123.19 125.095) (width 0.25) (layer F.Cu) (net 14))
 (segment (start 121.285 98.425) (end 121.285 123.19) (width 0.25) (layer F.Cu) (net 14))
 (segment (start 120.015 97.155) (end 121.285 98.425) (width 0.25) (layer F.Cu) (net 14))
 (segment (start 118.11 99.695) (end 120.65 102.235) (width 0.25) (layer F.Cu) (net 15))
 (segment (start 154.305 111.76) (end 156.21 109.855) (width 0.25) (layer F.Cu) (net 15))
 (segment (start 154.305 125.095) (end 154.305 111.76) (width 0.25) (layer F.Cu) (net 15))
 (segment (start 153.67 125.73) (end 154.305 125.095) (width 0.25) (layer F.Cu) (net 15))
 (segment (start 122.555 125.73) (end 153.67 125.73) (width 0.25) (layer F.Cu) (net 15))
 (segment (start 120.65 123.825) (end 122.555 125.73) (width 0.25) (layer F.Cu) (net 15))
 (segment (start 120.65 102.235) (end 120.65 123.825) (width 0.25) (layer F.Cu) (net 15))
 (segment (start 118.11 102.235) (end 123.19 107.315) (width 0.25) (layer B.Cu) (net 16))
 (segment (start 143.51 112.395) (end 140.97 109.855) (width 0.25) (layer B.Cu) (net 16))
 (segment (start 143.51 120.015) (end 143.51 112.395) (width 0.25) (layer B.Cu) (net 16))
 (segment (start 141.605 121.92) (end 143.51 120.015) (width 0.25) (layer B.Cu) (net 16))
 (segment (start 127.635 121.92) (end 141.605 121.92) (width 0.25) (layer B.Cu) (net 16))
 (segment (start 123.19 117.475) (end 127.635 121.92) (width 0.25) (layer B.Cu) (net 16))
 (segment (start 123.19 107.315) (end 123.19 117.475) (width 0.25) (layer B.Cu) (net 16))
 (segment (start 118.11 104.775) (end 122.555 109.22) (width 0.25) (layer B.Cu) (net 17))
 (segment (start 144.145 107.95) (end 140.97 104.775) (width 0.25) (layer B.Cu) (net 17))
 (segment (start 144.145 120.65) (end 144.145 107.95) (width 0.25) (layer B.Cu) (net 17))
 (segment (start 142.24 122.555) (end 144.145 120.65) (width 0.25) (layer B.Cu) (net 17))
 (segment (start 127 122.555) (end 142.24 122.555) (width 0.25) (layer B.Cu) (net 17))
 (segment (start 122.555 118.11) (end 127 122.555) (width 0.25) (layer B.Cu) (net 17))
 (segment (start 122.555 109.22) (end 122.555 118.11) (width 0.25) (layer B.Cu) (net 17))
 (segment (start 118.11 107.315) (end 121.92 111.125) (width 0.25) (layer B.Cu) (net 18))
 (segment (start 144.78 103.505) (end 140.97 99.695) (width 0.25) (layer B.Cu) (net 18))
 (segment (start 144.78 121.285) (end 144.78 103.505) (width 0.25) (layer B.Cu) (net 18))
 (segment (start 142.875 123.19) (end 144.78 121.285) (width 0.25) (layer B.Cu) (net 18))
 (segment (start 126.365 123.19) (end 142.875 123.19) (width 0.25) (layer B.Cu) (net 18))
 (segment (start 121.92 118.745) (end 126.365 123.19) (width 0.25) (layer B.Cu) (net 18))
 (segment (start 121.92 111.125) (end 121.92 118.745) (width 0.25) (layer B.Cu) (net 18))
 (segment (start 118.11 109.855) (end 121.285 113.03) (width 0.25) (layer B.Cu) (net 19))
 (segment (start 145.415 99.06) (end 140.97 94.615) (width 0.25) (layer B.Cu) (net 19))
 (segment (start 145.415 121.92) (end 145.415 99.06) (width 0.25) (layer B.Cu) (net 19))
 (segment (start 143.51 123.825) (end 145.415 121.92) (width 0.25) (layer B.Cu) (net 19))
 (segment (start 125.73 123.825) (end 143.51 123.825) (width 0.25) (layer B.Cu) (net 19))
 (segment (start 121.285 119.38) (end 125.73 123.825) (width 0.25) (layer B.Cu) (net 19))
 (segment (start 121.285 113.03) (end 121.285 119.38) (width 0.25) (layer B.Cu) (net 19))
 (segment (start 118.11 112.395) (end 120.65 114.935) (width 0.25) (layer B.Cu) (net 20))
 (segment (start 146.05 97.155) (end 140.97 92.075) (width 0.25) (layer B.Cu) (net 20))
 (segment (start 146.05 122.555) (end 146.05 97.155) (width 0.25) (layer B.Cu) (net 20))
 (segment (start 144.145 124.46) (end 146.05 122.555) (width 0.25) (layer B.Cu) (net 20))
 (segment (start 125.095 124.46) (end 144.145 124.46) (width 0.25) (layer B.Cu) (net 20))
 (segment (start 120.65 120.015) (end 125.095 124.46) (width 0.25) (layer B.Cu) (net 20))
 (segment (start 120.65 114.935) (end 120.65 120.015) (width 0.25) (layer B.Cu) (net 20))
 (segment (start 133.35 112.395) (end 135.255 114.3) (width 0.25) (layer F.Cu) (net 21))
 (segment (start 142.875 86.36) (end 140.97 84.455) (width 0.25) (layer F.Cu) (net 21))
 (segment (start 142.875 113.665) (end 142.875 86.36) (width 0.25) (layer F.Cu) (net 21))
 (segment (start 142.24 114.3) (end 142.875 113.665) (width 0.25) (layer F.Cu) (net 21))
 (segment (start 135.255 114.3) (end 142.24 114.3) (width 0.25) (layer F.Cu) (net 21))
 (segment (start 133.35 109.855) (end 139.065 104.14) (width 0.25) (layer F.Cu) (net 22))
 (segment (start 139.065 83.82) (end 140.97 81.915) (width 0.25) (layer F.Cu) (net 22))
 (segment (start 139.065 104.14) (end 139.065 83.82) (width 0.25) (layer F.Cu) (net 22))
 (segment (start 133.35 107.315) (end 138.43 102.235) (width 0.25) (layer F.Cu) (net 23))
 (segment (start 138.43 81.915) (end 140.97 79.375) (width 0.25) (layer F.Cu) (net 23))
 (segment (start 138.43 102.235) (end 138.43 81.915) (width 0.25) (layer F.Cu) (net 23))
 (segment (start 133.35 104.775) (end 137.795 100.33) (width 0.25) (layer F.Cu) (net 24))
 (segment (start 137.795 80.01) (end 140.97 76.835) (width 0.25) (layer F.Cu) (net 24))
 (segment (start 137.795 100.33) (end 137.795 80.01) (width 0.25) (layer F.Cu) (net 24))
 (segment (start 133.35 102.235) (end 137.16 98.425) (width 0.25) (layer F.Cu) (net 25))
 (segment (start 137.16 78.105) (end 140.97 74.295) (width 0.25) (layer F.Cu) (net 25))
 (segment (start 137.16 98.425) (end 137.16 78.105) (width 0.25) (layer F.Cu) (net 25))
 (segment (start 133.35 99.695) (end 136.525 96.52) (width 0.25) (layer F.Cu) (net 26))
 (segment (start 136.525 76.2) (end 140.97 71.755) (width 0.25) (layer F.Cu) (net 26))
 (segment (start 136.525 96.52) (end 136.525 76.2) (width 0.25) (layer F.Cu) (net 26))
 (segment (start 133.35 97.155) (end 135.89 94.615) (width 0.25) (layer F.Cu) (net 27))
 (segment (start 135.89 74.295) (end 140.97 69.215) (width 0.25) (layer F.Cu) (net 27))
 (segment (start 135.89 94.615) (end 135.89 74.295) (width 0.25) (layer F.Cu) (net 27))
 (segment (start 133.35 94.615) (end 135.255 92.71) (width 0.25) (layer F.Cu) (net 28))
 (segment (start 135.255 72.39) (end 140.97 66.675) (width 0.25) (layer F.Cu) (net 28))
 (segment (start 135.255 92.71) (end 135.255 72.39) (width 0.25) (layer F.Cu) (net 28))
 (segment (start 133.35 92.075) (end 131.445 93.98) (width 0.25) (layer F.Cu) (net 29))
 (segment (start 143.51 76.835) (end 156.21 64.135) (width 0.25) (layer F.Cu) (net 29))
 (segment (start 143.51 114.3) (end 143.51 76.835) (width 0.25) (layer F.Cu) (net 29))
 (segment (start 142.875 114.935) (end 143.51 114.3) (width 0.25) (layer F.Cu) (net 29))
 (segment (start 133.35 114.935) (end 142.875 114.935) (width 0.25) (layer F.Cu) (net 29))
 (segment (start 131.445 113.03) (end 133.35 114.935) (width 0.25) (layer F.Cu) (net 29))
 (segment (start 131.445 93.98) (end 131.445 113.03) (width 0.25) (layer F.Cu) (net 29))
 (segment (start 133.35 89.535) (end 134.62 88.265) (width 0.25) (layer F.Cu) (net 30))
 (segment (start 153.035 86.36) (end 156.21 89.535) (width 0.25) (layer B.Cu) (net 30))
 (segment (start 153.035 73.025) (end 153.035 86.36) (width 0.25) (layer B.Cu) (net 30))
 (segment (start 142.24 62.23) (end 153.035 73.025) (width 0.25) (layer B.Cu) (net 30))
 (segment (start 139.7 62.23) (end 142.24 62.23) (width 0.25) (layer B.Cu) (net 30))
 (segment (start 137.16 64.77) (end 139.7 62.23) (width 0.25) (layer B.Cu) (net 30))
 (segment (start 137.16 67.31) (end 137.16 64.77) (width 0.25) (layer B.Cu) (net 30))
 (via (at 137.16 67.31) (size 0.6) (drill 0.4) (layers F.Cu B.Cu) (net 30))
 (segment (start 134.62 69.85) (end 137.16 67.31) (width 0.25) (layer F.Cu) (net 30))
 (segment (start 134.62 88.265) (end 134.62 69.85) (width 0.25) (layer F.Cu) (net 30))
 (segment (start 133.35 86.995) (end 130.81 89.535) (width 0.25) (layer F.Cu) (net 31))
 (segment (start 144.145 78.74) (end 156.21 66.675) (width 0.25) (layer F.Cu) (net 31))
 (segment (start 144.145 114.935) (end 144.145 78.74) (width 0.25) (layer F.Cu) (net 31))
 (segment (start 143.51 115.57) (end 144.145 114.935) (width 0.25) (layer F.Cu) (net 31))
 (segment (start 132.715 115.57) (end 143.51 115.57) (width 0.25) (layer F.Cu) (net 31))
 (segment (start 130.81 113.665) (end 132.715 115.57) (width 0.25) (layer F.Cu) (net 31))
 (segment (start 130.81 89.535) (end 130.81 113.665) (width 0.25) (layer F.Cu) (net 31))
 (segment (start 133.35 84.455) (end 130.175 87.63) (width 0.25) (layer F.Cu) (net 32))
 (segment (start 144.78 80.645) (end 156.21 69.215) (width 0.25) (layer F.Cu) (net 32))
 (segment (start 144.78 115.57) (end 144.78 80.645) (width 0.25) (layer F.Cu) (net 32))
 (segment (start 144.145 116.205) (end 144.78 115.57) (width 0.25) (layer F.Cu) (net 32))
 (segment (start 132.08 116.205) (end 144.145 116.205) (width 0.25) (layer F.Cu) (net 32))
 (segment (start 130.175 114.3) (end 132.08 116.205) (width 0.25) (layer F.Cu) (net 32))
 (segment (start 130.175 87.63) (end 130.175 114.3) (width 0.25) (layer F.Cu) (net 32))
 (segment (start 133.35 81.915) (end 129.54 85.725) (width 0.25) (layer F.Cu) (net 33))
 (segment (start 145.415 82.55) (end 156.21 71.755) (width 0.25) (layer F.Cu) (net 33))
 (segment (start 145.415 116.205) (end 145.415 82.55) (width 0.25) (layer F.Cu) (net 33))
 (segment (start 144.78 116.84) (end 145.415 116.205) (width 0.25) (layer F.Cu) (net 33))
 (segment (start 131.445 116.84) (end 144.78 116.84) (width 0.25) (layer F.Cu) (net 33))
 (segment (start 129.54 114.935) (end 131.445 116.84) (width 0.25) (layer F.Cu) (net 33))
 (segment (start 129.54 85.725) (end 129.54 114.935) (width 0.25) (layer F.Cu) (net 33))
 (segment (start 133.35 79.375) (end 128.905 83.82) (width 0.25) (layer F.Cu) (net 34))
 (segment (start 146.05 84.455) (end 156.21 74.295) (width 0.25) (layer F.Cu) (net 34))
 (segment (start 146.05 116.84) (end 146.05 84.455) (width 0.25) (layer F.Cu) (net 34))
 (segment (start 145.415 117.475) (end 146.05 116.84) (width 0.25) (layer F.Cu) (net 34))
 (segment (start 130.81 117.475) (end 145.415 117.475) (width 0.25) (layer F.Cu) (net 34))
 (segment (start 128.905 115.57) (end 130.81 117.475) (width 0.25) (layer F.Cu) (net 34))
 (segment (start 128.905 83.82) (end 128.905 115.57) (width 0.25) (layer F.Cu) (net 34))
 (segment (start 133.35 76.835) (end 128.27 81.915) (width 0.25) (layer F.Cu) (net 35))
 (segment (start 146.685 86.36) (end 156.21 76.835) (width 0.25) (layer F.Cu) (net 35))
 (segment (start 146.685 117.475) (end 146.685 86.36) (width 0.25) (layer F.Cu) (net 35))
 (segment (start 146.05 118.11) (end 146.685 117.475) (width 0.25) (layer F.Cu) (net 35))
 (segment (start 130.175 118.11) (end 146.05 118.11) (width 0.25) (layer F.Cu) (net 35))
 (segment (start 128.27 116.205) (end 130.175 118.11) (width 0.25) (layer F.Cu) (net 35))
 (segment (start 128.27 81.915) (end 128.27 116.205) (width 0.25) (layer F.Cu) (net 35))
 (segment (start 133.35 74.295) (end 127.635 80.01) (width 0.25) (layer F.Cu) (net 36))
 (segment (start 147.32 88.265) (end 156.21 79.375) (width 0.25) (layer F.Cu) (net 36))
 (segment (start 147.32 118.11) (end 147.32 88.265) (width 0.25) (layer F.Cu) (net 36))
 (segment (start 146.685 118.745) (end 147.32 118.11) (width 0.25) (layer F.Cu) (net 36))
 (segment (start 129.54 118.745) (end 146.685 118.745) (width 0.25) (layer F.Cu) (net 36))
 (segment (start 127.635 116.84) (end 129.54 118.745) (width 0.25) (layer F.Cu) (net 36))
 (segment (start 127.635 80.01) (end 127.635 116.84) (width 0.25) (layer F.Cu) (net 36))
 (segment (start 133.35 71.755) (end 127 78.105) (width 0.25) (layer F.Cu) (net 37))
 (segment (start 147.955 90.17) (end 156.21 81.915) (width 0.25) (layer F.Cu) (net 37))
 (segment (start 147.955 118.745) (end 147.955 90.17) (width 0.25) (layer F.Cu) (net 37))
 (segment (start 147.32 119.38) (end 147.955 118.745) (width 0.25) (layer F.Cu) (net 37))
 (segment (start 128.905 119.38) (end 147.32 119.38) (width 0.25) (layer F.Cu) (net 37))
 (segment (start 127 117.475) (end 128.905 119.38) (width 0.25) (layer F.Cu) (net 37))
 (segment (start 127 78.105) (end 127 117.475) (width 0.25) (layer F.Cu) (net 37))
 (segment (start 133.35 69.215) (end 126.365 76.2) (width 0.25) (layer F.Cu) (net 38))
 (segment (start 148.59 92.075) (end 156.21 84.455) (width 0.25) (layer F.Cu) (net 38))
 (segment (start 148.59 119.38) (end 148.59 92.075) (width 0.25) (layer F.Cu) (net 38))
 (segment (start 147.955 120.015) (end 148.59 119.38) (width 0.25) (layer F.Cu) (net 38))
 (segment (start 128.27 120.015) (end 147.955 120.015) (width 0.25) (layer F.Cu) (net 38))
 (segment (start 126.365 118.11) (end 128.27 120.015) (width 0.25) (layer F.Cu) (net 38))
 (segment (start 126.365 76.2) (end 126.365 118.11) (width 0.25) (layer F.Cu) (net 38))
 (segment (start 133.35 66.675) (end 135.255 66.675) (width 0.25) (layer F.Cu) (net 39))
 (segment (start 137.795 64.135) (end 140.97 64.135) (width 0.25) (layer F.Cu) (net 39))
 (segment (start 135.255 66.675) (end 137.795 64.135) (width 0.25) (layer F.Cu) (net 39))
 (segment (start 133.35 64.135) (end 136.525 64.135) (width 0.25) (layer F.Cu) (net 40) (status 400000))
 (segment (start 142.24 62.23) (end 147.955 67.945) (width 0.25) (layer F.Cu) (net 40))
 (segment (start 147.955 67.945) (end 147.955 69.85) (width 0.25) (layer F.Cu) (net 40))
 (via (at 147.955 69.85) (size 0.6) (drill 0.4) (layers F.Cu B.Cu) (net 40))
 (segment (start 147.955 69.85) (end 147.955 111.76) (width 0.25) (layer B.Cu) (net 40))
 (segment (start 153.035 115.57) (end 156.21 112.395) (width 0.25) (layer B.Cu) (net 40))
 (segment (start 151.765 115.57) (end 153.035 115.57) (width 0.25) (layer B.Cu) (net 40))
 (segment (start 147.955 111.76) (end 151.765 115.57) (width 0.25) (layer B.Cu) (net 40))
 (segment (start 139.7 62.23) (end 142.24 62.23) (width 0.25) (layer F.Cu) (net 40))
 (segment (start 138.43 63.5) (end 139.7 62.23) (width 0.25) (layer F.Cu) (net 40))
 (segment (start 137.16 63.5) (end 138.43 63.5) (width 0.25) (layer F.Cu) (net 40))
 (segment (start 136.525 64.135) (end 137.16 63.5) (width 0.25) (layer F.Cu) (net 40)))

